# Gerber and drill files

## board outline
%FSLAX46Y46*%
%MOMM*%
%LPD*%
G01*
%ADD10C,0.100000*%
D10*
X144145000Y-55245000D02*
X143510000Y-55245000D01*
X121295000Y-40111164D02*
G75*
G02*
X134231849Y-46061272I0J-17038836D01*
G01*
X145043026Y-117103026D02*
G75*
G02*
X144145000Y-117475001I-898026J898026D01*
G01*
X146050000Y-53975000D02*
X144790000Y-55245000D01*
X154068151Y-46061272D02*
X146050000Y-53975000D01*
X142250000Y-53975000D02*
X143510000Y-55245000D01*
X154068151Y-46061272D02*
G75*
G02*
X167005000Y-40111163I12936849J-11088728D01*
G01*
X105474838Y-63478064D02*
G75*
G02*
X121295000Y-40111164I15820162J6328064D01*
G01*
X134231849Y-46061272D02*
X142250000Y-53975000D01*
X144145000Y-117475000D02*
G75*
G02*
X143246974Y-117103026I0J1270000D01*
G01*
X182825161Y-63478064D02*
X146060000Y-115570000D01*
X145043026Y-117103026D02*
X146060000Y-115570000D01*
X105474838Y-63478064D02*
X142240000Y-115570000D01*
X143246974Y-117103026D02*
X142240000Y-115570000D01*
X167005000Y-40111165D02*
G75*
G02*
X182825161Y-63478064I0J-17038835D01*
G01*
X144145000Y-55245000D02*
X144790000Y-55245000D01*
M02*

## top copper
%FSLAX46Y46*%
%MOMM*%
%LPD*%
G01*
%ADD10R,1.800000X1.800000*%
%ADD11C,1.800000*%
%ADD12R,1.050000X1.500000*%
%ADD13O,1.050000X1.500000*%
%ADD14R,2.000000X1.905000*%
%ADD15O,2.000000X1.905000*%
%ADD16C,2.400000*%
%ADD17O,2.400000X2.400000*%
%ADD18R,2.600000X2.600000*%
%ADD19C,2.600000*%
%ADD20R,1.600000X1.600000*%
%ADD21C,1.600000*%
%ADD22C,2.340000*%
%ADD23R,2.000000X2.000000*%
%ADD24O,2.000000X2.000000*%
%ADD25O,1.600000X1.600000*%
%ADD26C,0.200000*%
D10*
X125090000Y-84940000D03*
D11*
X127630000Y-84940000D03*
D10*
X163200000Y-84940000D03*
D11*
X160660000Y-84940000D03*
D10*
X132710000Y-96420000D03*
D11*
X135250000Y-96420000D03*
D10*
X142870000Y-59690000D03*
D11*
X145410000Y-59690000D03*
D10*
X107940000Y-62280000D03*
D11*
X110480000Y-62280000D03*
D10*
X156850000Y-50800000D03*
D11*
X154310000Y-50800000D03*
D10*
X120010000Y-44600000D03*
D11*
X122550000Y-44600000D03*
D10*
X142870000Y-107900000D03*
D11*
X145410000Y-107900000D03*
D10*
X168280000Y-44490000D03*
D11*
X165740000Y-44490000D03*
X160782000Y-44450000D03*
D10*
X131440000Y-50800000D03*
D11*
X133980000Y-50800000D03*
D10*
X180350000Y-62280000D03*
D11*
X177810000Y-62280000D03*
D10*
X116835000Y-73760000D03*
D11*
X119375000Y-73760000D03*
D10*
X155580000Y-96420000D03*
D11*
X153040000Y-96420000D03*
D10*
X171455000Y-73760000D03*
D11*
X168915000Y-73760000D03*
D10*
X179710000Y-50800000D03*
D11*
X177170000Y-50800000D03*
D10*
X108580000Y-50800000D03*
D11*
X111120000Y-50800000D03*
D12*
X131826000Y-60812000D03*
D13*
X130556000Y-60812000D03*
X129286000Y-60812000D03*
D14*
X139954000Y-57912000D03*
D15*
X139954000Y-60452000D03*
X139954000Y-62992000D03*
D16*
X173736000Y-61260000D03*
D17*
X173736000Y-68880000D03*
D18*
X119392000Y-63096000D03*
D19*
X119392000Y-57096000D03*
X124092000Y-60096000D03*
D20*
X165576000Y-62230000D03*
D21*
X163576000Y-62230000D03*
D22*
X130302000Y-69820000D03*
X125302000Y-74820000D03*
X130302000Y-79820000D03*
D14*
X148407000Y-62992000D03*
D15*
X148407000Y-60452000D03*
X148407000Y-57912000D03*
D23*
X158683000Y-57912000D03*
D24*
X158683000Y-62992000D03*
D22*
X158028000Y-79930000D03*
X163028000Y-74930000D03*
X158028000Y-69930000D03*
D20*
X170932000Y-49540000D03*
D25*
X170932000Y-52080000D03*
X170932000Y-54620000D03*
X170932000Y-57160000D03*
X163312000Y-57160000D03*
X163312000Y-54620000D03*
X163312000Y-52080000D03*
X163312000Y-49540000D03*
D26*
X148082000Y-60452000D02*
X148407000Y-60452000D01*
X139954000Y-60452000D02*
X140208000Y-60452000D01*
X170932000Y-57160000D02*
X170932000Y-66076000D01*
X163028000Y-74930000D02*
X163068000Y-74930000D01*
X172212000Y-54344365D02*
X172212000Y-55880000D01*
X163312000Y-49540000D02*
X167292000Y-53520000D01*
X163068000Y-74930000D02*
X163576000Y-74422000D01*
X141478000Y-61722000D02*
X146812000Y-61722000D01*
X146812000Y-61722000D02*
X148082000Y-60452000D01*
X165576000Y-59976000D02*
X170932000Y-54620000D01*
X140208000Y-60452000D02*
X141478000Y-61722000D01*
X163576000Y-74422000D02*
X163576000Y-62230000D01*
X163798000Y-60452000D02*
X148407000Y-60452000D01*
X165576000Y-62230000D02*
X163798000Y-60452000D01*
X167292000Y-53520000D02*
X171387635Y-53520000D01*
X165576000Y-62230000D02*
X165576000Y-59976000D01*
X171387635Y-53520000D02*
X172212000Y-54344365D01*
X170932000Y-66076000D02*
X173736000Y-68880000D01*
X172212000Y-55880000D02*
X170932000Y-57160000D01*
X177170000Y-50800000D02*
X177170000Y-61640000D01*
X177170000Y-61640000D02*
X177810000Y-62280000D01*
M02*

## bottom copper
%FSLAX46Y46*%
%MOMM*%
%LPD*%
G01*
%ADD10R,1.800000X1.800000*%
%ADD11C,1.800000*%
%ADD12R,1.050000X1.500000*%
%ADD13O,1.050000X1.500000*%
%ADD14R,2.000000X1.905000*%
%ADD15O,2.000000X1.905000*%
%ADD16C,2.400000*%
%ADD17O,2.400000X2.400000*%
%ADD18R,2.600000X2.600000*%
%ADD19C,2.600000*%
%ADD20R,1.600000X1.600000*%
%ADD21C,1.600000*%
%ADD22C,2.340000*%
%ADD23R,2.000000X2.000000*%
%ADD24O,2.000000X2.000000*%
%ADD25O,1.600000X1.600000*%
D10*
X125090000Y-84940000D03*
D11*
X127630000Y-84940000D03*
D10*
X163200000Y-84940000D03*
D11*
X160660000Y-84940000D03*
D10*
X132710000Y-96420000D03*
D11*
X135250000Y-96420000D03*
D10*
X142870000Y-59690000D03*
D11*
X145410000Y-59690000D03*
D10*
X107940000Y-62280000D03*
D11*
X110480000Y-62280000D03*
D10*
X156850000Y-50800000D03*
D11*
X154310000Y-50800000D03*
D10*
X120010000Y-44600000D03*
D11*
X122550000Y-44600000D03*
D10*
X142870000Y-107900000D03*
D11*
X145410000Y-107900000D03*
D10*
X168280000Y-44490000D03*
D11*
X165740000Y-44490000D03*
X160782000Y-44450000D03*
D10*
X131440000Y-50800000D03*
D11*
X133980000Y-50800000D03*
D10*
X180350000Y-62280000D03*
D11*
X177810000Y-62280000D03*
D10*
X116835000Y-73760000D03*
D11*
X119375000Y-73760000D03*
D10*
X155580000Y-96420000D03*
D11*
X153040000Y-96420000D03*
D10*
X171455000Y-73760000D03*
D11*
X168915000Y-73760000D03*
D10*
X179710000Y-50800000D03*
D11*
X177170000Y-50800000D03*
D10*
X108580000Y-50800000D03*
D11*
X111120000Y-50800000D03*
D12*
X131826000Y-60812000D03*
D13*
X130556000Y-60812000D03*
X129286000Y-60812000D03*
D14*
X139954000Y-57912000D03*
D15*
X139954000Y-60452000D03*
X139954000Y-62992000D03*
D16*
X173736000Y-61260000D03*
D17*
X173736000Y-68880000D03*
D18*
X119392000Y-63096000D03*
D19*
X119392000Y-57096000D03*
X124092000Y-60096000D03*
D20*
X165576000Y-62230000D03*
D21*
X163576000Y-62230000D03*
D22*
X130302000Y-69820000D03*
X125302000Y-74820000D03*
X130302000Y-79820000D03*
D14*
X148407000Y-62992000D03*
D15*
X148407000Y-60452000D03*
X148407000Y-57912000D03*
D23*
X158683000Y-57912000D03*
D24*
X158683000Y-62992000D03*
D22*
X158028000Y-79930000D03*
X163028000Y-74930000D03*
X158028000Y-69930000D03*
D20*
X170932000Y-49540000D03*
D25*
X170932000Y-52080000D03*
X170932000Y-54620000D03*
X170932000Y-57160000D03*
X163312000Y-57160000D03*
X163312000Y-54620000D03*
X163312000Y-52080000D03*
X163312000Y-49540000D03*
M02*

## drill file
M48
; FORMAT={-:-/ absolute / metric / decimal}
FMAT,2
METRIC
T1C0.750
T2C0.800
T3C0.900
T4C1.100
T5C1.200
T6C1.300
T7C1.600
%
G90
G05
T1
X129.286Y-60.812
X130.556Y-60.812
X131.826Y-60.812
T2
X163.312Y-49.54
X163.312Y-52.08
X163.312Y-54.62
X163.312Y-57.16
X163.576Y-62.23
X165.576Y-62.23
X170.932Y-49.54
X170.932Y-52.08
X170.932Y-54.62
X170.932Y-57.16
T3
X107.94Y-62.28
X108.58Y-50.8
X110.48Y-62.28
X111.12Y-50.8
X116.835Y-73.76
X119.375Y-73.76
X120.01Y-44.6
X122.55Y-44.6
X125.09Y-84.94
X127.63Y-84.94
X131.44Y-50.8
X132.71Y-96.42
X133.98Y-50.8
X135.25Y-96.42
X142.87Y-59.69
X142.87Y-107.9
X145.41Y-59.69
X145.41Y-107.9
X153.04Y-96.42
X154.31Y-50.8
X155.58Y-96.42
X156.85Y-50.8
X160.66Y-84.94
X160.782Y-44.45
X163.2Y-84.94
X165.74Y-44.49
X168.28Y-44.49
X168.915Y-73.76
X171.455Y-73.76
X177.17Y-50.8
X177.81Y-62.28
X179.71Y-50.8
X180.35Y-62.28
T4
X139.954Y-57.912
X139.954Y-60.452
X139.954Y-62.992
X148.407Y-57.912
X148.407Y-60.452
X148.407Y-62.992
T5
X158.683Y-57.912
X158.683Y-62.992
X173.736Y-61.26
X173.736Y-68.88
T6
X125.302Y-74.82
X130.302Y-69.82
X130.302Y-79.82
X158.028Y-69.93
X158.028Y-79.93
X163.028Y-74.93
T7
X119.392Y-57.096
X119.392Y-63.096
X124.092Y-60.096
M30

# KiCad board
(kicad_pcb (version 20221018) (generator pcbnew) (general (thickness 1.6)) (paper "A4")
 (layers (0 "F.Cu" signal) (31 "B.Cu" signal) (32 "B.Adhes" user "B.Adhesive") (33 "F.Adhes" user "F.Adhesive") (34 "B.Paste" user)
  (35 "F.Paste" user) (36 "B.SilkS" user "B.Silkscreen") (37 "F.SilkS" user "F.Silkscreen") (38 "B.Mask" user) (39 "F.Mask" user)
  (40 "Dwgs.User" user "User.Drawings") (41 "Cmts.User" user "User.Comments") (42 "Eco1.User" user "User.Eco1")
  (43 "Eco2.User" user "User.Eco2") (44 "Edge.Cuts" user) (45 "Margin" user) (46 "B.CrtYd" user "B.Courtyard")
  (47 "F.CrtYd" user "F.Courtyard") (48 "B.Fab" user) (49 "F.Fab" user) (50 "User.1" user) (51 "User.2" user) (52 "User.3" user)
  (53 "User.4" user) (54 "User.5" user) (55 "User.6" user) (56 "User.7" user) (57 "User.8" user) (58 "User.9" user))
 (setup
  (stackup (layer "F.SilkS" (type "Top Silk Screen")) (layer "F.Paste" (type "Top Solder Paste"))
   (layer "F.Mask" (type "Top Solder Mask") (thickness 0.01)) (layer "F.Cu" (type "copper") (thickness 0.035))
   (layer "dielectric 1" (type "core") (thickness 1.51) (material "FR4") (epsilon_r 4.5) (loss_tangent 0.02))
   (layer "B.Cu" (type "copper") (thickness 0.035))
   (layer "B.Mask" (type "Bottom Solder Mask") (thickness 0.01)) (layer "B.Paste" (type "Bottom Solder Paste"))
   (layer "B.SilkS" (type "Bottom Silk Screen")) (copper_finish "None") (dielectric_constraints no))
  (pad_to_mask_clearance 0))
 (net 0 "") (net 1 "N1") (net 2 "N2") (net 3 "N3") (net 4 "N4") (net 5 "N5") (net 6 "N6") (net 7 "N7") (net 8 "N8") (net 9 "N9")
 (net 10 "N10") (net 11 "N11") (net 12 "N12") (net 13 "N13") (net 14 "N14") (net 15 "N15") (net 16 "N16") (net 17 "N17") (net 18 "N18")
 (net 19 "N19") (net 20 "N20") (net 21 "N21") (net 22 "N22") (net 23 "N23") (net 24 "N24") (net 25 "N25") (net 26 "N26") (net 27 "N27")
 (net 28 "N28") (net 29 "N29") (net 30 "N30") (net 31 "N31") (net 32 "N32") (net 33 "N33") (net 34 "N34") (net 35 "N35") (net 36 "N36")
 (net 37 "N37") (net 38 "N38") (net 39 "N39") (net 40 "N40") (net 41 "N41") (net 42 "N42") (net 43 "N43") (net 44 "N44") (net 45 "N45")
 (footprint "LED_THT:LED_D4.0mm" (layer "F.Cu") (at 125.09 84.94)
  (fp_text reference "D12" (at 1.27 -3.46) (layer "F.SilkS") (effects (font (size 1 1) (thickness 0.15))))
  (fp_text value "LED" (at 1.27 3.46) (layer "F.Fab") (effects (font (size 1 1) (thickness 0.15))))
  (pad "1" thru_hole rect (at 0 0) (size 1.8 1.8) (drill 0.9) (layers "*.Cu" "*.Mask") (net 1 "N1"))
  (pad "2" thru_hole circle (at 2.54 0) (size 1.8 1.8) (drill 0.9) (layers "*.Cu" "*.Mask") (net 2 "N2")))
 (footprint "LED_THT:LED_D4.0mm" (layer "F.Cu") (at 163.2 84.94 180)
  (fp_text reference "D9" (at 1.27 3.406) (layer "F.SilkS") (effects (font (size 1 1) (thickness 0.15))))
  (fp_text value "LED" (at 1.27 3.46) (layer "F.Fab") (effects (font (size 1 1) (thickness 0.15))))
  (pad "1" thru_hole rect (at 0 0 180) (size 1.8 1.8) (drill 0.9) (layers "*.Cu" "*.Mask") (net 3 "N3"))
  (pad "2" thru_hole circle (at 2.54 0 180) (size 1.8 1.8) (drill 0.9) (layers "*.Cu" "*.Mask") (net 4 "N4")))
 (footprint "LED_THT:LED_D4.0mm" (layer "F.Cu") (at 132.71 96.42)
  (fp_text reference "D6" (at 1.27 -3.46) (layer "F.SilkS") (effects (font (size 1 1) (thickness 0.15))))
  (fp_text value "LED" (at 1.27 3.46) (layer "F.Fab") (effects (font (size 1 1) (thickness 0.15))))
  (pad "1" thru_hole rect (at 0 0) (size 1.8 1.8) (drill 0.9) (layers "*.Cu" "*.Mask") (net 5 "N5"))
  (pad "2" thru_hole circle (at 2.54 0) (size 1.8 1.8) (drill 0.9) (layers "*.Cu" "*.Mask") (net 4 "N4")))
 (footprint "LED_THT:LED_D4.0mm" (layer "F.Cu") (at 142.87 59.69)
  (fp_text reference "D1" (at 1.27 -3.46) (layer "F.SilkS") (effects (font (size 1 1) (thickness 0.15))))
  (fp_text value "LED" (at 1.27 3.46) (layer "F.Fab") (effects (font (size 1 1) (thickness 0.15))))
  (pad "1" thru_hole rect (at 0 0) (size 1.8 1.8) (drill 0.9) (layers "*.Cu" "*.Mask") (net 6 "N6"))
  (pad "2" thru_hole circle (at 2.54 0) (size 1.8 1.8) (drill 0.9) (layers "*.Cu" "*.Mask") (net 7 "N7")))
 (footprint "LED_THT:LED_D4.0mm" (layer "F.Cu") (at 107.94 62.28)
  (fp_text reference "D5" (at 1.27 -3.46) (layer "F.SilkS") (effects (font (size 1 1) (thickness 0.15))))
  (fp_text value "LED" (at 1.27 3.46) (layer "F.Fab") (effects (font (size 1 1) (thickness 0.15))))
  (pad "1" thru_hole rect (at 0 0) (size 1.8 1.8) (drill 0.9) (layers "*.Cu" "*.Mask") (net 3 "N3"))
  (pad "2" thru_hole circle (at 2.54 0) (size 1.8 1.8) (drill 0.9) (layers "*.Cu" "*.Mask") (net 2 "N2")))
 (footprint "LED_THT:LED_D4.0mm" (layer "F.Cu") (at 156.85 50.8 180)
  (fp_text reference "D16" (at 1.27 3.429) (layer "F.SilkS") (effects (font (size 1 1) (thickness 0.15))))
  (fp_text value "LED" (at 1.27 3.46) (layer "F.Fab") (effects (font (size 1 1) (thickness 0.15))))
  (pad "1" thru_hole rect (at 0 0 180) (size 1.8 1.8) (drill 0.9) (layers "*.Cu" "*.Mask") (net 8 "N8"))
  (pad "2" thru_hole circle (at 2.54 0 180) (size 1.8 1.8) (drill 0.9) (layers "*.Cu" "*.Mask") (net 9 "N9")))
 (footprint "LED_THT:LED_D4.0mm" (layer "F.Cu") (at 120.01 44.6)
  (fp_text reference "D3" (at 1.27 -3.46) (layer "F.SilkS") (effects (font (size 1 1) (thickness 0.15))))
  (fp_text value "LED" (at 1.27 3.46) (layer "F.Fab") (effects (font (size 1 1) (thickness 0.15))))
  (pad "1" thru_hole rect (at 0 0) (size 1.8 1.8) (drill 0.9) (layers "*.Cu" "*.Mask") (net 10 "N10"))
  (pad "2" thru_hole circle (at 2.54 0) (size 1.8 1.8) (drill 0.9) (layers "*.Cu" "*.Mask") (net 2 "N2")))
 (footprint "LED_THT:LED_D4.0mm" (layer "F.Cu") (at 142.87 107.9)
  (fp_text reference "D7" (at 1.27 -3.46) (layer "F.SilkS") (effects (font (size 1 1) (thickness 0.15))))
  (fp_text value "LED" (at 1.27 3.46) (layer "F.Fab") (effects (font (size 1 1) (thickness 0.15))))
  (pad "1" thru_hole rect (at 0 0) (size 1.8 1.8) (drill 0.9) (layers "*.Cu" "*.Mask") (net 10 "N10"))
  (pad "2" thru_hole circle (at 2.54 0) (size 1.8 1.8) (drill 0.9) (layers "*.Cu" "*.Mask") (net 4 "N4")))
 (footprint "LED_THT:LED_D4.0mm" (layer "F.Cu") (at 168.28 44.49 180)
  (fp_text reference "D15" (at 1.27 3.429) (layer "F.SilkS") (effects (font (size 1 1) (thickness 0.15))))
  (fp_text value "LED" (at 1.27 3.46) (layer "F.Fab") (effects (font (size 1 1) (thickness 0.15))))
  (pad "1" thru_hole rect (at 0 0 180) (size 1.8 1.8) (drill 0.9) (layers "*.Cu" "*.Mask") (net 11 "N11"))
  (pad "2" thru_hole circle (at 2.54 0 180) (size 1.8 1.8) (drill 0.9) (layers "*.Cu" "*.Mask") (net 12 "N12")))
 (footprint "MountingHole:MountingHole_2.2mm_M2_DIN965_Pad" (layer "F.Cu") (at 160.782 44.45)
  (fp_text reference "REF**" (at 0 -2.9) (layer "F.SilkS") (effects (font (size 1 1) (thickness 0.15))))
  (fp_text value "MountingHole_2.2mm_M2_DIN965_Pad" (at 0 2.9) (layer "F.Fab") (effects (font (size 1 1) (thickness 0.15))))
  (pad "1" thru_hole circle (at 0 0) (size 1.8 1.8) (drill 0.9) (layers "*.Cu" "*.Mask")))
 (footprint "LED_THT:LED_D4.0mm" (layer "F.Cu") (at 131.44 50.8)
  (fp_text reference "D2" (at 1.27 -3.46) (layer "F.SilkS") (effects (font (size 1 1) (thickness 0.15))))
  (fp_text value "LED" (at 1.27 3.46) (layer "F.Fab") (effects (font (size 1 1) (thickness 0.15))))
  (pad "1" thru_hole rect (at 0 0) (size 1.8 1.8) (drill 0.9) (layers "*.Cu" "*.Mask") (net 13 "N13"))
  (pad "2" thru_hole circle (at 2.54 0) (size 1.8 1.8) (drill 0.9) (layers "*.Cu" "*.Mask") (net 2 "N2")))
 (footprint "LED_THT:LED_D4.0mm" (layer "F.Cu") (at 180.35 62.28 180)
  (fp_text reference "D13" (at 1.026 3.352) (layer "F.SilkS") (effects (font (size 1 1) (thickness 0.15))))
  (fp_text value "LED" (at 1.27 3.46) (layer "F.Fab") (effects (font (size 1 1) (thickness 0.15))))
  (pad "1" thru_hole rect (at 0 0 180) (size 1.8 1.8) (drill 0.9) (layers "*.Cu" "*.Mask") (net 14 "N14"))
  (pad "2" thru_hole circle (at 2.54 0 180) (size 1.8 1.8) (drill 0.9) (layers "*.Cu" "*.Mask") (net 4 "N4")))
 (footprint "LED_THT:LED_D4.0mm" (layer "F.Cu") (at 116.835 73.76)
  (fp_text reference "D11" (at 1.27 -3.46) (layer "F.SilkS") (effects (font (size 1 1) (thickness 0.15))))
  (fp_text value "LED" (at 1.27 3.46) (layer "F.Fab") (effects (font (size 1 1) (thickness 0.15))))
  (pad "1" thru_hole rect (at 0 0) (size 1.8 1.8) (drill 0.9) (layers "*.Cu" "*.Mask") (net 14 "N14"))
  (pad "2" thru_hole circle (at 2.54 0) (size 1.8 1.8) (drill 0.9) (layers "*.Cu" "*.Mask") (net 2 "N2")))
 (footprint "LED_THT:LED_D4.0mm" (layer "F.Cu") (at 155.58 96.42 180)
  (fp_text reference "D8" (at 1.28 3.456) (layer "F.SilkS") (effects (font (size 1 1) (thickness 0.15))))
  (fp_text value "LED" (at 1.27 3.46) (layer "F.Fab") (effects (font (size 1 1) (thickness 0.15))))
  (pad "1" thru_hole rect (at 0 0 180) (size 1.8 1.8) (drill 0.9) (layers "*.Cu" "*.Mask") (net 13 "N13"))
  (pad "2" thru_hole circle (at 2.54 0 180) (size 1.8 1.8) (drill 0.9) (layers "*.Cu" "*.Mask") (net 4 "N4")))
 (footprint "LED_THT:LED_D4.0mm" (layer "F.Cu") (at 171.455 73.76 180)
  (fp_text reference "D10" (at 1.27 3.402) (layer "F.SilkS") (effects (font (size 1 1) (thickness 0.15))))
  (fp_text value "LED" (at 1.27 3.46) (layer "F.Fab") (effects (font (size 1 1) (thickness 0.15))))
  (pad "1" thru_hole rect (at 0 0 180) (size 1.8 1.8) (drill 0.9) (layers "*.Cu" "*.Mask") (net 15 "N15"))
  (pad "2" thru_hole circle (at 2.54 0 180) (size 1.8 1.8) (drill 0.9) (layers "*.Cu" "*.Mask") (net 4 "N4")))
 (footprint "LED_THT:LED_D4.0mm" (layer "F.Cu") (at 179.71 50.8 180)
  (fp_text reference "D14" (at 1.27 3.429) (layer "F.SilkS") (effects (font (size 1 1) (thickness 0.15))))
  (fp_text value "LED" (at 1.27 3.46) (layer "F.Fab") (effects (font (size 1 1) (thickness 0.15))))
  (pad "1" thru_hole rect (at 0 0 180) (size 1.8 1.8) (drill 0.9) (layers "*.Cu" "*.Mask") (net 1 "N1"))
  (pad "2" thru_hole circle (at 2.54 0 180) (size 1.8 1.8) (drill 0.9) (layers "*.Cu" "*.Mask") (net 4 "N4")))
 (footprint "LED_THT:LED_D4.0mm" (layer "F.Cu") (at 108.58 50.8)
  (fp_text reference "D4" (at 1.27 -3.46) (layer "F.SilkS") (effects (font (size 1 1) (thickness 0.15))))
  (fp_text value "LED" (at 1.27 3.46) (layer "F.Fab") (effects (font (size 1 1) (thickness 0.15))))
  (pad "1" thru_hole rect (at 0 0) (size 1.8 1.8) (drill 0.9) (layers "*.Cu" "*.Mask") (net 5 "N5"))
  (pad "2" thru_hole circle (at 2.54 0) (size 1.8 1.8) (drill 0.9) (layers "*.Cu" "*.Mask") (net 2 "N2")))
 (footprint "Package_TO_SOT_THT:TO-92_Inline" (layer "B.Cu") (at 131.826 60.812 180)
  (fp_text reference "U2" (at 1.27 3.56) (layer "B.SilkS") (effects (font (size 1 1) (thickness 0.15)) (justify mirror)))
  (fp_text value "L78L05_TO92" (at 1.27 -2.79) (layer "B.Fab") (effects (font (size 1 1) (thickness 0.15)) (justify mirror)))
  (pad "1" thru_hole rect (at 0 0 180) (size 1.05 1.5) (drill 0.75) (layers "*.Cu" "*.Mask") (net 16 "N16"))
  (pad "2" thru_hole oval (at 1.27 0 180) (size 1.05 1.5) (drill 0.75) (layers "*.Cu" "*.Mask") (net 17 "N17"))
  (pad "3" thru_hole oval (at 2.54 0 180) (size 1.05 1.5) (drill 0.75) (layers "*.Cu" "*.Mask") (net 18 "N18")))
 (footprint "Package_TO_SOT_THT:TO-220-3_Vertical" (layer "B.Cu") (at 139.954 57.912 -90)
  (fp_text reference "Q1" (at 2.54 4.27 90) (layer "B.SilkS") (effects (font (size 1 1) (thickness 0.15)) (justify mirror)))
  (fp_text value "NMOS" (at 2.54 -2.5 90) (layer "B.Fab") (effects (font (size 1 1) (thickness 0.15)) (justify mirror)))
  (pad "1" thru_hole rect (at 0 0 270) (size 1.905 2) (drill 1.1) (layers "*.Cu" "*.Mask") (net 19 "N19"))
  (pad "2" thru_hole oval (at 2.54 0 270) (size 1.905 2) (drill 1.1) (layers "*.Cu" "*.Mask") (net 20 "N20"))
  (pad "3" thru_hole oval (at 5.08 0 270) (size 1.905 2) (drill 1.1) (layers "*.Cu" "*.Mask") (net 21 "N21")))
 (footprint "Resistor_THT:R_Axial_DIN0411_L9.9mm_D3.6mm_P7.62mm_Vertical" (layer "B.Cu") (at 173.736 61.26 -90)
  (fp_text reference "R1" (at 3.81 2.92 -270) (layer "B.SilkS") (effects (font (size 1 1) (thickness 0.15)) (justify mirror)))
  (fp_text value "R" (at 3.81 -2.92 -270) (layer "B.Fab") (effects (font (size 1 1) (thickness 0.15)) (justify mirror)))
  (pad "1" thru_hole circle (at 0 0 270) (size 2.4 2.4) (drill 1.2) (layers "*.Cu" "*.Mask") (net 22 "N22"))
  (pad "2" thru_hole oval (at 7.62 0 270) (size 2.4 2.4) (drill 1.2) (layers "*.Cu" "*.Mask") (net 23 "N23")))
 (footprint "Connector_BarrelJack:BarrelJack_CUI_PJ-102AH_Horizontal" (layer "B.Cu") (at 119.392 63.096)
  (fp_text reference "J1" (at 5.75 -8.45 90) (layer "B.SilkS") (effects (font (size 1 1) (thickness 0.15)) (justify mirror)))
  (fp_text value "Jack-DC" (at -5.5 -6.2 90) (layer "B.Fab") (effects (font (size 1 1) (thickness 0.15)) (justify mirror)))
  (pad "1" thru_hole rect (at 0 0) (size 2.6 2.6) (drill 1.6) (layers "*.Cu" "*.Mask") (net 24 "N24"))
  (pad "2" thru_hole circle (at 0 -6) (size 2.6 2.6) (drill 1.6) (layers "*.Cu" "*.Mask") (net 15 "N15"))
  (pad "3" thru_hole circle (at 4.7 -3) (size 2.6 2.6) (drill 1.6) (layers "*.Cu" "*.Mask")))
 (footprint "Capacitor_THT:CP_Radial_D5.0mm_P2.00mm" (layer "B.Cu") (at 165.576 62.23 180)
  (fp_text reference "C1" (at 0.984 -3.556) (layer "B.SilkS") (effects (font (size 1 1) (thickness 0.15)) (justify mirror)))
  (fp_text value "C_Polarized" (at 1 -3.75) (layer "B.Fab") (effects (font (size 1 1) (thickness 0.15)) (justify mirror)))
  (pad "1" thru_hole rect (at 0 0 180) (size 1.6 1.6) (drill 0.8) (layers "*.Cu" "*.Mask") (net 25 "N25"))
  (pad "2" thru_hole circle (at 2 0 180) (size 1.6 1.6) (drill 0.8) (layers "*.Cu" "*.Mask") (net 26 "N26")))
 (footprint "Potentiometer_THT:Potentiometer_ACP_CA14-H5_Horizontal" (layer "B.Cu") (at 130.302 69.82 180)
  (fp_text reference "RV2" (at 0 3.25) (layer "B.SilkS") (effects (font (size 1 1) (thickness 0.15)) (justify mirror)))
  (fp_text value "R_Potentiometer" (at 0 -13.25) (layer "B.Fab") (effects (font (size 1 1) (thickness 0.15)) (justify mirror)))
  (pad "1" thru_hole circle (at 0 0 180) (size 2.34 2.34) (drill 1.3) (layers "*.Cu" "*.Mask") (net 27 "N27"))
  (pad "2" thru_hole circle (at 5 -5 180) (size 2.34 2.34) (drill 1.3) (layers "*.Cu" "*.Mask") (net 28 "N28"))
  (pad "3" thru_hole circle (at 0 -10 180) (size 2.34 2.34) (drill 1.3) (layers "*.Cu" "*.Mask") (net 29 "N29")))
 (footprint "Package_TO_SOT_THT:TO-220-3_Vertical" (layer "B.Cu") (at 148.407 62.992 90)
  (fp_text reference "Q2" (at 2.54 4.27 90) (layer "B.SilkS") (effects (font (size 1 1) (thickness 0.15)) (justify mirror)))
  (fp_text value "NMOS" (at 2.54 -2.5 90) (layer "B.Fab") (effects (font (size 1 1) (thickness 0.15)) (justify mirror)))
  (pad "1" thru_hole rect (at 0 0 90) (size 1.905 2) (drill 1.1) (layers "*.Cu" "*.Mask") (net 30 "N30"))
  (pad "2" thru_hole oval (at 2.54 0 90) (size 1.905 2) (drill 1.1) (layers "*.Cu" "*.Mask") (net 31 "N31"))
  (pad "3" thru_hole oval (at 5.08 0 90) (size 1.905 2) (drill 1.1) (layers "*.Cu" "*.Mask") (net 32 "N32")))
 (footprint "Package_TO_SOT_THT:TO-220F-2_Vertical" (layer "B.Cu") (at 158.683 57.912 -90)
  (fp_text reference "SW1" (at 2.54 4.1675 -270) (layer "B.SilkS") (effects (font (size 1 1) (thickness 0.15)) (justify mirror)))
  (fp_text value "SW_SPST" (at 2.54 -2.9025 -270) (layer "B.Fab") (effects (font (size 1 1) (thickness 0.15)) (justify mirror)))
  (pad "1" thru_hole rect (at 0 0 270) (size 2 2) (drill 1.2) (layers "*.Cu" "*.Mask") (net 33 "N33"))
  (pad "2" thru_hole oval (at 5.08 0 270) (size 2 2) (drill 1.2) (layers "*.Cu" "*.Mask") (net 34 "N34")))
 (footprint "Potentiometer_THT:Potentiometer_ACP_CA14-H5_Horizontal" (layer "B.Cu") (at 158.028 79.93)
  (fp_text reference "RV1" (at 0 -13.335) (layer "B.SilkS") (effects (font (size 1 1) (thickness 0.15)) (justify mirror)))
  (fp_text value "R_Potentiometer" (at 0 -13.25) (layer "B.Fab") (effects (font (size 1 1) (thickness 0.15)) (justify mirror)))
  (pad "1" thru_hole circle (at 0 0) (size 2.34 2.34) (drill 1.3) (layers "*.Cu" "*.Mask") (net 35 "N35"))
  (pad "2" thru_hole circle (at 5 -5) (size 2.34 2.34) (drill 1.3) (layers "*.Cu" "*.Mask") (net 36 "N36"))
  (pad "3" thru_hole circle (at 0 -10) (size 2.34 2.34) (drill 1.3) (layers "*.Cu" "*.Mask") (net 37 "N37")))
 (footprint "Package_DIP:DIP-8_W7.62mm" (layer "B.Cu") (at 170.932 49.54 180)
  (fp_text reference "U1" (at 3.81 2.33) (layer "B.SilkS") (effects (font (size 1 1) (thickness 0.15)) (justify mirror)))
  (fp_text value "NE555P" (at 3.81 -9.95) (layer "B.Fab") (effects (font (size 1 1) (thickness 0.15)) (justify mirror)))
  (pad "1" thru_hole rect (at 0 0 180) (size 1.6 1.6) (drill 0.8) (layers "*.Cu" "*.Mask") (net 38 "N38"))
  (pad "2" thru_hole oval (at 0 -2.54 180) (size 1.6 1.6) (drill 0.8) (layers "*.Cu" "*.Mask") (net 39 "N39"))
  (pad "3" thru_hole oval (at 0 -5.08 180) (size 1.6 1.6) (drill 0.8) (layers "*.Cu" "*.Mask") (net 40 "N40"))
  (pad "4" thru_hole oval (at 0 -7.62 180) (size 1.6 1.6) (drill 0.8) (layers "*.Cu" "*.Mask") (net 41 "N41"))
  (pad "5" thru_hole oval (at 7.62 -7.62 180) (size 1.6 1.6) (drill 0.8) (layers "*.Cu" "*.Mask") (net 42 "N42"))
  (pad "6" thru_hole oval (at 7.62 -5.08 180) (size 1.6 1.6) (drill 0.8) (layers "*.Cu" "*.Mask") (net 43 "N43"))
  (pad "7" thru_hole oval (at 7.62 -2.54 180) (size 1.6 1.6) (drill 0.8) (layers "*.Cu" "*.Mask") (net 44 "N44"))
  (pad "8" thru_hole oval (at 7.62 0 180) (size 1.6 1.6) (drill 0.8) (layers "*.Cu" "*.Mask") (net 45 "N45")))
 (gr_line locked (start 144.145 55.245) (end 143.51 55.245) (stroke (width 0.1) (type default)) (layer "Edge.Cuts"))
 (gr_arc locked (start 121.295 40.111164) (mid 128.414792 41.67) (end 134.231849 46.061272) (stroke (width 0.1) (type default))
  (layer "Edge.Cuts"))
 (gr_arc locked (start 145.043026 117.103026) (mid 144.631008 117.378328) (end 144.145 117.475) (stroke (width 0.1) (type default))
  (layer "Edge.Cuts"))
 (gr_line locked (start 146.05 53.975) (end 144.79 55.245) (stroke (width 0.1) (type default)) (layer "Edge.Cuts"))
 (gr_line locked (start 154.068151 46.061272) (end 146.05 53.975) (stroke (width 0.1) (type default)) (layer "Edge.Cuts"))
 (gr_line locked (start 142.25 53.975) (end 143.51 55.245) (stroke (width 0.1) (type default)) (layer "Edge.Cuts"))
 (gr_arc locked (start 154.068151 46.061272) (mid 159.885208 41.67) (end 167.005 40.111164) (stroke (width 0.1) (type default))
  (layer "Edge.Cuts"))
 (gr_arc locked (start 105.474838 63.478064) (mid 107.185699 47.597538) (end 121.295 40.111164) (stroke (width 0.1) (type default))
  (layer "Edge.Cuts"))
 (gr_line locked (start 134.231849 46.061272) (end 142.25 53.975) (stroke (width 0.1) (type default)) (layer "Edge.Cuts"))
 (gr_arc locked (start 144.145 117.475) (mid 143.658992 117.378327) (end 143.246974 117.103026) (stroke (width 0.1) (type default))
  (layer "Edge.Cuts"))
 (gr_line locked (start 182.825161 63.478064) (end 146.06 115.57) (stroke (width 0.1) (type default)) (layer "Edge.Cuts"))
 (gr_line locked (start 145.043026 117.103026) (end 146.06 115.57) (stroke (width 0.1) (type default)) (layer "Edge.Cuts"))
 (gr_line locked (start 105.474838 63.478064) (end 142.24 115.57) (stroke (width 0.1) (type default)) (layer "Edge.Cuts"))
 (gr_line locked (start 143.246974 117.103026) (end 142.24 115.57) (stroke (width 0.1) (type default)) (layer "Edge.Cuts"))
 (gr_arc locked (start 167.005 40.111165) (mid 181.114301 47.597538) (end 182.825161 63.478064) (stroke (width 0.1) (type default))
  (layer "Edge.Cuts"))
 (gr_line locked (start 144.145 55.245) (end 144.79 55.245) (stroke (width 0.1) (type default)) (layer "Edge.Cuts"))
 (segment (start 148.082 60.452) (end 148.407 60.452) (width 0.2) (layer "F.Cu") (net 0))
 (segment (start 139.954 60.452) (end 140.208 60.452) (width 0.2) (layer "F.Cu") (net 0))
 (segment (start 170.932 57.16) (end 170.932 66.076) (width 0.2) (layer "F.Cu") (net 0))
 (segment (start 163.028 74.93) (end 163.068 74.93) (width 0.2) (layer "F.Cu") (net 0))
 (segment (start 172.212 54.344365) (end 172.212 55.88) (width 0.2) (layer "F.Cu") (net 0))
 (segment (start 163.312 49.54) (end 167.292 53.52) (width 0.2) (layer "F.Cu") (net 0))
 (segment (start 163.068 74.93) (end 163.576 74.422) (width 0.2) (layer "F.Cu") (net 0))
 (segment (start 141.478 61.722) (end 146.812 61.722) (width 0.2) (layer "F.Cu") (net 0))
 (segment (start 146.812 61.722) (end 148.082 60.452) (width 0.2) (layer "F.Cu") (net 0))
 (segment (start 165.576 59.976) (end 170.932 54.62) (width 0.2) (layer "F.Cu") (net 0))
 (segment (start 140.208 60.452) (end 141.478 61.722) (width 0.2) (layer "F.Cu") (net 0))
 (segment (start 163.576 74.422) (end 163.576 62.23) (width 0.2) (layer "F.Cu") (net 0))
 (segment (start 163.798 60.452) (end 148.407 60.452) (width 0.2) (layer "F.Cu") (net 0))
 (segment (start 165.576 62.23) (end 163.798 60.452) (width 0.2) (layer "F.Cu") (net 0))
 (segment (start 167.292 53.52) (end 171.387635 53.52) (width 0.2) (layer "F.Cu") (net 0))
 (segment (start 165.576 62.23) (end 165.576 59.976) (width 0.2) (layer "F.Cu") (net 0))
 (segment (start 171.387635 53.52) (end 172.212 54.344365) (width 0.2) (layer "F.Cu") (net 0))
 (segment (start 170.932 66.076) (end 173.736 68.88) (width 0.2) (layer "F.Cu") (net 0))
 (segment (start 172.212 55.88) (end 170.932 57.16) (width 0.2) (layer "F.Cu") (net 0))
 (segment (start 177.17 50.8) (end 177.17 61.64) (width 0.2) (layer "F.Cu") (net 4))
 (segment (start 177.17 61.64) (end 177.81 62.28) (width 0.2) (layer "F.Cu") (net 4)))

